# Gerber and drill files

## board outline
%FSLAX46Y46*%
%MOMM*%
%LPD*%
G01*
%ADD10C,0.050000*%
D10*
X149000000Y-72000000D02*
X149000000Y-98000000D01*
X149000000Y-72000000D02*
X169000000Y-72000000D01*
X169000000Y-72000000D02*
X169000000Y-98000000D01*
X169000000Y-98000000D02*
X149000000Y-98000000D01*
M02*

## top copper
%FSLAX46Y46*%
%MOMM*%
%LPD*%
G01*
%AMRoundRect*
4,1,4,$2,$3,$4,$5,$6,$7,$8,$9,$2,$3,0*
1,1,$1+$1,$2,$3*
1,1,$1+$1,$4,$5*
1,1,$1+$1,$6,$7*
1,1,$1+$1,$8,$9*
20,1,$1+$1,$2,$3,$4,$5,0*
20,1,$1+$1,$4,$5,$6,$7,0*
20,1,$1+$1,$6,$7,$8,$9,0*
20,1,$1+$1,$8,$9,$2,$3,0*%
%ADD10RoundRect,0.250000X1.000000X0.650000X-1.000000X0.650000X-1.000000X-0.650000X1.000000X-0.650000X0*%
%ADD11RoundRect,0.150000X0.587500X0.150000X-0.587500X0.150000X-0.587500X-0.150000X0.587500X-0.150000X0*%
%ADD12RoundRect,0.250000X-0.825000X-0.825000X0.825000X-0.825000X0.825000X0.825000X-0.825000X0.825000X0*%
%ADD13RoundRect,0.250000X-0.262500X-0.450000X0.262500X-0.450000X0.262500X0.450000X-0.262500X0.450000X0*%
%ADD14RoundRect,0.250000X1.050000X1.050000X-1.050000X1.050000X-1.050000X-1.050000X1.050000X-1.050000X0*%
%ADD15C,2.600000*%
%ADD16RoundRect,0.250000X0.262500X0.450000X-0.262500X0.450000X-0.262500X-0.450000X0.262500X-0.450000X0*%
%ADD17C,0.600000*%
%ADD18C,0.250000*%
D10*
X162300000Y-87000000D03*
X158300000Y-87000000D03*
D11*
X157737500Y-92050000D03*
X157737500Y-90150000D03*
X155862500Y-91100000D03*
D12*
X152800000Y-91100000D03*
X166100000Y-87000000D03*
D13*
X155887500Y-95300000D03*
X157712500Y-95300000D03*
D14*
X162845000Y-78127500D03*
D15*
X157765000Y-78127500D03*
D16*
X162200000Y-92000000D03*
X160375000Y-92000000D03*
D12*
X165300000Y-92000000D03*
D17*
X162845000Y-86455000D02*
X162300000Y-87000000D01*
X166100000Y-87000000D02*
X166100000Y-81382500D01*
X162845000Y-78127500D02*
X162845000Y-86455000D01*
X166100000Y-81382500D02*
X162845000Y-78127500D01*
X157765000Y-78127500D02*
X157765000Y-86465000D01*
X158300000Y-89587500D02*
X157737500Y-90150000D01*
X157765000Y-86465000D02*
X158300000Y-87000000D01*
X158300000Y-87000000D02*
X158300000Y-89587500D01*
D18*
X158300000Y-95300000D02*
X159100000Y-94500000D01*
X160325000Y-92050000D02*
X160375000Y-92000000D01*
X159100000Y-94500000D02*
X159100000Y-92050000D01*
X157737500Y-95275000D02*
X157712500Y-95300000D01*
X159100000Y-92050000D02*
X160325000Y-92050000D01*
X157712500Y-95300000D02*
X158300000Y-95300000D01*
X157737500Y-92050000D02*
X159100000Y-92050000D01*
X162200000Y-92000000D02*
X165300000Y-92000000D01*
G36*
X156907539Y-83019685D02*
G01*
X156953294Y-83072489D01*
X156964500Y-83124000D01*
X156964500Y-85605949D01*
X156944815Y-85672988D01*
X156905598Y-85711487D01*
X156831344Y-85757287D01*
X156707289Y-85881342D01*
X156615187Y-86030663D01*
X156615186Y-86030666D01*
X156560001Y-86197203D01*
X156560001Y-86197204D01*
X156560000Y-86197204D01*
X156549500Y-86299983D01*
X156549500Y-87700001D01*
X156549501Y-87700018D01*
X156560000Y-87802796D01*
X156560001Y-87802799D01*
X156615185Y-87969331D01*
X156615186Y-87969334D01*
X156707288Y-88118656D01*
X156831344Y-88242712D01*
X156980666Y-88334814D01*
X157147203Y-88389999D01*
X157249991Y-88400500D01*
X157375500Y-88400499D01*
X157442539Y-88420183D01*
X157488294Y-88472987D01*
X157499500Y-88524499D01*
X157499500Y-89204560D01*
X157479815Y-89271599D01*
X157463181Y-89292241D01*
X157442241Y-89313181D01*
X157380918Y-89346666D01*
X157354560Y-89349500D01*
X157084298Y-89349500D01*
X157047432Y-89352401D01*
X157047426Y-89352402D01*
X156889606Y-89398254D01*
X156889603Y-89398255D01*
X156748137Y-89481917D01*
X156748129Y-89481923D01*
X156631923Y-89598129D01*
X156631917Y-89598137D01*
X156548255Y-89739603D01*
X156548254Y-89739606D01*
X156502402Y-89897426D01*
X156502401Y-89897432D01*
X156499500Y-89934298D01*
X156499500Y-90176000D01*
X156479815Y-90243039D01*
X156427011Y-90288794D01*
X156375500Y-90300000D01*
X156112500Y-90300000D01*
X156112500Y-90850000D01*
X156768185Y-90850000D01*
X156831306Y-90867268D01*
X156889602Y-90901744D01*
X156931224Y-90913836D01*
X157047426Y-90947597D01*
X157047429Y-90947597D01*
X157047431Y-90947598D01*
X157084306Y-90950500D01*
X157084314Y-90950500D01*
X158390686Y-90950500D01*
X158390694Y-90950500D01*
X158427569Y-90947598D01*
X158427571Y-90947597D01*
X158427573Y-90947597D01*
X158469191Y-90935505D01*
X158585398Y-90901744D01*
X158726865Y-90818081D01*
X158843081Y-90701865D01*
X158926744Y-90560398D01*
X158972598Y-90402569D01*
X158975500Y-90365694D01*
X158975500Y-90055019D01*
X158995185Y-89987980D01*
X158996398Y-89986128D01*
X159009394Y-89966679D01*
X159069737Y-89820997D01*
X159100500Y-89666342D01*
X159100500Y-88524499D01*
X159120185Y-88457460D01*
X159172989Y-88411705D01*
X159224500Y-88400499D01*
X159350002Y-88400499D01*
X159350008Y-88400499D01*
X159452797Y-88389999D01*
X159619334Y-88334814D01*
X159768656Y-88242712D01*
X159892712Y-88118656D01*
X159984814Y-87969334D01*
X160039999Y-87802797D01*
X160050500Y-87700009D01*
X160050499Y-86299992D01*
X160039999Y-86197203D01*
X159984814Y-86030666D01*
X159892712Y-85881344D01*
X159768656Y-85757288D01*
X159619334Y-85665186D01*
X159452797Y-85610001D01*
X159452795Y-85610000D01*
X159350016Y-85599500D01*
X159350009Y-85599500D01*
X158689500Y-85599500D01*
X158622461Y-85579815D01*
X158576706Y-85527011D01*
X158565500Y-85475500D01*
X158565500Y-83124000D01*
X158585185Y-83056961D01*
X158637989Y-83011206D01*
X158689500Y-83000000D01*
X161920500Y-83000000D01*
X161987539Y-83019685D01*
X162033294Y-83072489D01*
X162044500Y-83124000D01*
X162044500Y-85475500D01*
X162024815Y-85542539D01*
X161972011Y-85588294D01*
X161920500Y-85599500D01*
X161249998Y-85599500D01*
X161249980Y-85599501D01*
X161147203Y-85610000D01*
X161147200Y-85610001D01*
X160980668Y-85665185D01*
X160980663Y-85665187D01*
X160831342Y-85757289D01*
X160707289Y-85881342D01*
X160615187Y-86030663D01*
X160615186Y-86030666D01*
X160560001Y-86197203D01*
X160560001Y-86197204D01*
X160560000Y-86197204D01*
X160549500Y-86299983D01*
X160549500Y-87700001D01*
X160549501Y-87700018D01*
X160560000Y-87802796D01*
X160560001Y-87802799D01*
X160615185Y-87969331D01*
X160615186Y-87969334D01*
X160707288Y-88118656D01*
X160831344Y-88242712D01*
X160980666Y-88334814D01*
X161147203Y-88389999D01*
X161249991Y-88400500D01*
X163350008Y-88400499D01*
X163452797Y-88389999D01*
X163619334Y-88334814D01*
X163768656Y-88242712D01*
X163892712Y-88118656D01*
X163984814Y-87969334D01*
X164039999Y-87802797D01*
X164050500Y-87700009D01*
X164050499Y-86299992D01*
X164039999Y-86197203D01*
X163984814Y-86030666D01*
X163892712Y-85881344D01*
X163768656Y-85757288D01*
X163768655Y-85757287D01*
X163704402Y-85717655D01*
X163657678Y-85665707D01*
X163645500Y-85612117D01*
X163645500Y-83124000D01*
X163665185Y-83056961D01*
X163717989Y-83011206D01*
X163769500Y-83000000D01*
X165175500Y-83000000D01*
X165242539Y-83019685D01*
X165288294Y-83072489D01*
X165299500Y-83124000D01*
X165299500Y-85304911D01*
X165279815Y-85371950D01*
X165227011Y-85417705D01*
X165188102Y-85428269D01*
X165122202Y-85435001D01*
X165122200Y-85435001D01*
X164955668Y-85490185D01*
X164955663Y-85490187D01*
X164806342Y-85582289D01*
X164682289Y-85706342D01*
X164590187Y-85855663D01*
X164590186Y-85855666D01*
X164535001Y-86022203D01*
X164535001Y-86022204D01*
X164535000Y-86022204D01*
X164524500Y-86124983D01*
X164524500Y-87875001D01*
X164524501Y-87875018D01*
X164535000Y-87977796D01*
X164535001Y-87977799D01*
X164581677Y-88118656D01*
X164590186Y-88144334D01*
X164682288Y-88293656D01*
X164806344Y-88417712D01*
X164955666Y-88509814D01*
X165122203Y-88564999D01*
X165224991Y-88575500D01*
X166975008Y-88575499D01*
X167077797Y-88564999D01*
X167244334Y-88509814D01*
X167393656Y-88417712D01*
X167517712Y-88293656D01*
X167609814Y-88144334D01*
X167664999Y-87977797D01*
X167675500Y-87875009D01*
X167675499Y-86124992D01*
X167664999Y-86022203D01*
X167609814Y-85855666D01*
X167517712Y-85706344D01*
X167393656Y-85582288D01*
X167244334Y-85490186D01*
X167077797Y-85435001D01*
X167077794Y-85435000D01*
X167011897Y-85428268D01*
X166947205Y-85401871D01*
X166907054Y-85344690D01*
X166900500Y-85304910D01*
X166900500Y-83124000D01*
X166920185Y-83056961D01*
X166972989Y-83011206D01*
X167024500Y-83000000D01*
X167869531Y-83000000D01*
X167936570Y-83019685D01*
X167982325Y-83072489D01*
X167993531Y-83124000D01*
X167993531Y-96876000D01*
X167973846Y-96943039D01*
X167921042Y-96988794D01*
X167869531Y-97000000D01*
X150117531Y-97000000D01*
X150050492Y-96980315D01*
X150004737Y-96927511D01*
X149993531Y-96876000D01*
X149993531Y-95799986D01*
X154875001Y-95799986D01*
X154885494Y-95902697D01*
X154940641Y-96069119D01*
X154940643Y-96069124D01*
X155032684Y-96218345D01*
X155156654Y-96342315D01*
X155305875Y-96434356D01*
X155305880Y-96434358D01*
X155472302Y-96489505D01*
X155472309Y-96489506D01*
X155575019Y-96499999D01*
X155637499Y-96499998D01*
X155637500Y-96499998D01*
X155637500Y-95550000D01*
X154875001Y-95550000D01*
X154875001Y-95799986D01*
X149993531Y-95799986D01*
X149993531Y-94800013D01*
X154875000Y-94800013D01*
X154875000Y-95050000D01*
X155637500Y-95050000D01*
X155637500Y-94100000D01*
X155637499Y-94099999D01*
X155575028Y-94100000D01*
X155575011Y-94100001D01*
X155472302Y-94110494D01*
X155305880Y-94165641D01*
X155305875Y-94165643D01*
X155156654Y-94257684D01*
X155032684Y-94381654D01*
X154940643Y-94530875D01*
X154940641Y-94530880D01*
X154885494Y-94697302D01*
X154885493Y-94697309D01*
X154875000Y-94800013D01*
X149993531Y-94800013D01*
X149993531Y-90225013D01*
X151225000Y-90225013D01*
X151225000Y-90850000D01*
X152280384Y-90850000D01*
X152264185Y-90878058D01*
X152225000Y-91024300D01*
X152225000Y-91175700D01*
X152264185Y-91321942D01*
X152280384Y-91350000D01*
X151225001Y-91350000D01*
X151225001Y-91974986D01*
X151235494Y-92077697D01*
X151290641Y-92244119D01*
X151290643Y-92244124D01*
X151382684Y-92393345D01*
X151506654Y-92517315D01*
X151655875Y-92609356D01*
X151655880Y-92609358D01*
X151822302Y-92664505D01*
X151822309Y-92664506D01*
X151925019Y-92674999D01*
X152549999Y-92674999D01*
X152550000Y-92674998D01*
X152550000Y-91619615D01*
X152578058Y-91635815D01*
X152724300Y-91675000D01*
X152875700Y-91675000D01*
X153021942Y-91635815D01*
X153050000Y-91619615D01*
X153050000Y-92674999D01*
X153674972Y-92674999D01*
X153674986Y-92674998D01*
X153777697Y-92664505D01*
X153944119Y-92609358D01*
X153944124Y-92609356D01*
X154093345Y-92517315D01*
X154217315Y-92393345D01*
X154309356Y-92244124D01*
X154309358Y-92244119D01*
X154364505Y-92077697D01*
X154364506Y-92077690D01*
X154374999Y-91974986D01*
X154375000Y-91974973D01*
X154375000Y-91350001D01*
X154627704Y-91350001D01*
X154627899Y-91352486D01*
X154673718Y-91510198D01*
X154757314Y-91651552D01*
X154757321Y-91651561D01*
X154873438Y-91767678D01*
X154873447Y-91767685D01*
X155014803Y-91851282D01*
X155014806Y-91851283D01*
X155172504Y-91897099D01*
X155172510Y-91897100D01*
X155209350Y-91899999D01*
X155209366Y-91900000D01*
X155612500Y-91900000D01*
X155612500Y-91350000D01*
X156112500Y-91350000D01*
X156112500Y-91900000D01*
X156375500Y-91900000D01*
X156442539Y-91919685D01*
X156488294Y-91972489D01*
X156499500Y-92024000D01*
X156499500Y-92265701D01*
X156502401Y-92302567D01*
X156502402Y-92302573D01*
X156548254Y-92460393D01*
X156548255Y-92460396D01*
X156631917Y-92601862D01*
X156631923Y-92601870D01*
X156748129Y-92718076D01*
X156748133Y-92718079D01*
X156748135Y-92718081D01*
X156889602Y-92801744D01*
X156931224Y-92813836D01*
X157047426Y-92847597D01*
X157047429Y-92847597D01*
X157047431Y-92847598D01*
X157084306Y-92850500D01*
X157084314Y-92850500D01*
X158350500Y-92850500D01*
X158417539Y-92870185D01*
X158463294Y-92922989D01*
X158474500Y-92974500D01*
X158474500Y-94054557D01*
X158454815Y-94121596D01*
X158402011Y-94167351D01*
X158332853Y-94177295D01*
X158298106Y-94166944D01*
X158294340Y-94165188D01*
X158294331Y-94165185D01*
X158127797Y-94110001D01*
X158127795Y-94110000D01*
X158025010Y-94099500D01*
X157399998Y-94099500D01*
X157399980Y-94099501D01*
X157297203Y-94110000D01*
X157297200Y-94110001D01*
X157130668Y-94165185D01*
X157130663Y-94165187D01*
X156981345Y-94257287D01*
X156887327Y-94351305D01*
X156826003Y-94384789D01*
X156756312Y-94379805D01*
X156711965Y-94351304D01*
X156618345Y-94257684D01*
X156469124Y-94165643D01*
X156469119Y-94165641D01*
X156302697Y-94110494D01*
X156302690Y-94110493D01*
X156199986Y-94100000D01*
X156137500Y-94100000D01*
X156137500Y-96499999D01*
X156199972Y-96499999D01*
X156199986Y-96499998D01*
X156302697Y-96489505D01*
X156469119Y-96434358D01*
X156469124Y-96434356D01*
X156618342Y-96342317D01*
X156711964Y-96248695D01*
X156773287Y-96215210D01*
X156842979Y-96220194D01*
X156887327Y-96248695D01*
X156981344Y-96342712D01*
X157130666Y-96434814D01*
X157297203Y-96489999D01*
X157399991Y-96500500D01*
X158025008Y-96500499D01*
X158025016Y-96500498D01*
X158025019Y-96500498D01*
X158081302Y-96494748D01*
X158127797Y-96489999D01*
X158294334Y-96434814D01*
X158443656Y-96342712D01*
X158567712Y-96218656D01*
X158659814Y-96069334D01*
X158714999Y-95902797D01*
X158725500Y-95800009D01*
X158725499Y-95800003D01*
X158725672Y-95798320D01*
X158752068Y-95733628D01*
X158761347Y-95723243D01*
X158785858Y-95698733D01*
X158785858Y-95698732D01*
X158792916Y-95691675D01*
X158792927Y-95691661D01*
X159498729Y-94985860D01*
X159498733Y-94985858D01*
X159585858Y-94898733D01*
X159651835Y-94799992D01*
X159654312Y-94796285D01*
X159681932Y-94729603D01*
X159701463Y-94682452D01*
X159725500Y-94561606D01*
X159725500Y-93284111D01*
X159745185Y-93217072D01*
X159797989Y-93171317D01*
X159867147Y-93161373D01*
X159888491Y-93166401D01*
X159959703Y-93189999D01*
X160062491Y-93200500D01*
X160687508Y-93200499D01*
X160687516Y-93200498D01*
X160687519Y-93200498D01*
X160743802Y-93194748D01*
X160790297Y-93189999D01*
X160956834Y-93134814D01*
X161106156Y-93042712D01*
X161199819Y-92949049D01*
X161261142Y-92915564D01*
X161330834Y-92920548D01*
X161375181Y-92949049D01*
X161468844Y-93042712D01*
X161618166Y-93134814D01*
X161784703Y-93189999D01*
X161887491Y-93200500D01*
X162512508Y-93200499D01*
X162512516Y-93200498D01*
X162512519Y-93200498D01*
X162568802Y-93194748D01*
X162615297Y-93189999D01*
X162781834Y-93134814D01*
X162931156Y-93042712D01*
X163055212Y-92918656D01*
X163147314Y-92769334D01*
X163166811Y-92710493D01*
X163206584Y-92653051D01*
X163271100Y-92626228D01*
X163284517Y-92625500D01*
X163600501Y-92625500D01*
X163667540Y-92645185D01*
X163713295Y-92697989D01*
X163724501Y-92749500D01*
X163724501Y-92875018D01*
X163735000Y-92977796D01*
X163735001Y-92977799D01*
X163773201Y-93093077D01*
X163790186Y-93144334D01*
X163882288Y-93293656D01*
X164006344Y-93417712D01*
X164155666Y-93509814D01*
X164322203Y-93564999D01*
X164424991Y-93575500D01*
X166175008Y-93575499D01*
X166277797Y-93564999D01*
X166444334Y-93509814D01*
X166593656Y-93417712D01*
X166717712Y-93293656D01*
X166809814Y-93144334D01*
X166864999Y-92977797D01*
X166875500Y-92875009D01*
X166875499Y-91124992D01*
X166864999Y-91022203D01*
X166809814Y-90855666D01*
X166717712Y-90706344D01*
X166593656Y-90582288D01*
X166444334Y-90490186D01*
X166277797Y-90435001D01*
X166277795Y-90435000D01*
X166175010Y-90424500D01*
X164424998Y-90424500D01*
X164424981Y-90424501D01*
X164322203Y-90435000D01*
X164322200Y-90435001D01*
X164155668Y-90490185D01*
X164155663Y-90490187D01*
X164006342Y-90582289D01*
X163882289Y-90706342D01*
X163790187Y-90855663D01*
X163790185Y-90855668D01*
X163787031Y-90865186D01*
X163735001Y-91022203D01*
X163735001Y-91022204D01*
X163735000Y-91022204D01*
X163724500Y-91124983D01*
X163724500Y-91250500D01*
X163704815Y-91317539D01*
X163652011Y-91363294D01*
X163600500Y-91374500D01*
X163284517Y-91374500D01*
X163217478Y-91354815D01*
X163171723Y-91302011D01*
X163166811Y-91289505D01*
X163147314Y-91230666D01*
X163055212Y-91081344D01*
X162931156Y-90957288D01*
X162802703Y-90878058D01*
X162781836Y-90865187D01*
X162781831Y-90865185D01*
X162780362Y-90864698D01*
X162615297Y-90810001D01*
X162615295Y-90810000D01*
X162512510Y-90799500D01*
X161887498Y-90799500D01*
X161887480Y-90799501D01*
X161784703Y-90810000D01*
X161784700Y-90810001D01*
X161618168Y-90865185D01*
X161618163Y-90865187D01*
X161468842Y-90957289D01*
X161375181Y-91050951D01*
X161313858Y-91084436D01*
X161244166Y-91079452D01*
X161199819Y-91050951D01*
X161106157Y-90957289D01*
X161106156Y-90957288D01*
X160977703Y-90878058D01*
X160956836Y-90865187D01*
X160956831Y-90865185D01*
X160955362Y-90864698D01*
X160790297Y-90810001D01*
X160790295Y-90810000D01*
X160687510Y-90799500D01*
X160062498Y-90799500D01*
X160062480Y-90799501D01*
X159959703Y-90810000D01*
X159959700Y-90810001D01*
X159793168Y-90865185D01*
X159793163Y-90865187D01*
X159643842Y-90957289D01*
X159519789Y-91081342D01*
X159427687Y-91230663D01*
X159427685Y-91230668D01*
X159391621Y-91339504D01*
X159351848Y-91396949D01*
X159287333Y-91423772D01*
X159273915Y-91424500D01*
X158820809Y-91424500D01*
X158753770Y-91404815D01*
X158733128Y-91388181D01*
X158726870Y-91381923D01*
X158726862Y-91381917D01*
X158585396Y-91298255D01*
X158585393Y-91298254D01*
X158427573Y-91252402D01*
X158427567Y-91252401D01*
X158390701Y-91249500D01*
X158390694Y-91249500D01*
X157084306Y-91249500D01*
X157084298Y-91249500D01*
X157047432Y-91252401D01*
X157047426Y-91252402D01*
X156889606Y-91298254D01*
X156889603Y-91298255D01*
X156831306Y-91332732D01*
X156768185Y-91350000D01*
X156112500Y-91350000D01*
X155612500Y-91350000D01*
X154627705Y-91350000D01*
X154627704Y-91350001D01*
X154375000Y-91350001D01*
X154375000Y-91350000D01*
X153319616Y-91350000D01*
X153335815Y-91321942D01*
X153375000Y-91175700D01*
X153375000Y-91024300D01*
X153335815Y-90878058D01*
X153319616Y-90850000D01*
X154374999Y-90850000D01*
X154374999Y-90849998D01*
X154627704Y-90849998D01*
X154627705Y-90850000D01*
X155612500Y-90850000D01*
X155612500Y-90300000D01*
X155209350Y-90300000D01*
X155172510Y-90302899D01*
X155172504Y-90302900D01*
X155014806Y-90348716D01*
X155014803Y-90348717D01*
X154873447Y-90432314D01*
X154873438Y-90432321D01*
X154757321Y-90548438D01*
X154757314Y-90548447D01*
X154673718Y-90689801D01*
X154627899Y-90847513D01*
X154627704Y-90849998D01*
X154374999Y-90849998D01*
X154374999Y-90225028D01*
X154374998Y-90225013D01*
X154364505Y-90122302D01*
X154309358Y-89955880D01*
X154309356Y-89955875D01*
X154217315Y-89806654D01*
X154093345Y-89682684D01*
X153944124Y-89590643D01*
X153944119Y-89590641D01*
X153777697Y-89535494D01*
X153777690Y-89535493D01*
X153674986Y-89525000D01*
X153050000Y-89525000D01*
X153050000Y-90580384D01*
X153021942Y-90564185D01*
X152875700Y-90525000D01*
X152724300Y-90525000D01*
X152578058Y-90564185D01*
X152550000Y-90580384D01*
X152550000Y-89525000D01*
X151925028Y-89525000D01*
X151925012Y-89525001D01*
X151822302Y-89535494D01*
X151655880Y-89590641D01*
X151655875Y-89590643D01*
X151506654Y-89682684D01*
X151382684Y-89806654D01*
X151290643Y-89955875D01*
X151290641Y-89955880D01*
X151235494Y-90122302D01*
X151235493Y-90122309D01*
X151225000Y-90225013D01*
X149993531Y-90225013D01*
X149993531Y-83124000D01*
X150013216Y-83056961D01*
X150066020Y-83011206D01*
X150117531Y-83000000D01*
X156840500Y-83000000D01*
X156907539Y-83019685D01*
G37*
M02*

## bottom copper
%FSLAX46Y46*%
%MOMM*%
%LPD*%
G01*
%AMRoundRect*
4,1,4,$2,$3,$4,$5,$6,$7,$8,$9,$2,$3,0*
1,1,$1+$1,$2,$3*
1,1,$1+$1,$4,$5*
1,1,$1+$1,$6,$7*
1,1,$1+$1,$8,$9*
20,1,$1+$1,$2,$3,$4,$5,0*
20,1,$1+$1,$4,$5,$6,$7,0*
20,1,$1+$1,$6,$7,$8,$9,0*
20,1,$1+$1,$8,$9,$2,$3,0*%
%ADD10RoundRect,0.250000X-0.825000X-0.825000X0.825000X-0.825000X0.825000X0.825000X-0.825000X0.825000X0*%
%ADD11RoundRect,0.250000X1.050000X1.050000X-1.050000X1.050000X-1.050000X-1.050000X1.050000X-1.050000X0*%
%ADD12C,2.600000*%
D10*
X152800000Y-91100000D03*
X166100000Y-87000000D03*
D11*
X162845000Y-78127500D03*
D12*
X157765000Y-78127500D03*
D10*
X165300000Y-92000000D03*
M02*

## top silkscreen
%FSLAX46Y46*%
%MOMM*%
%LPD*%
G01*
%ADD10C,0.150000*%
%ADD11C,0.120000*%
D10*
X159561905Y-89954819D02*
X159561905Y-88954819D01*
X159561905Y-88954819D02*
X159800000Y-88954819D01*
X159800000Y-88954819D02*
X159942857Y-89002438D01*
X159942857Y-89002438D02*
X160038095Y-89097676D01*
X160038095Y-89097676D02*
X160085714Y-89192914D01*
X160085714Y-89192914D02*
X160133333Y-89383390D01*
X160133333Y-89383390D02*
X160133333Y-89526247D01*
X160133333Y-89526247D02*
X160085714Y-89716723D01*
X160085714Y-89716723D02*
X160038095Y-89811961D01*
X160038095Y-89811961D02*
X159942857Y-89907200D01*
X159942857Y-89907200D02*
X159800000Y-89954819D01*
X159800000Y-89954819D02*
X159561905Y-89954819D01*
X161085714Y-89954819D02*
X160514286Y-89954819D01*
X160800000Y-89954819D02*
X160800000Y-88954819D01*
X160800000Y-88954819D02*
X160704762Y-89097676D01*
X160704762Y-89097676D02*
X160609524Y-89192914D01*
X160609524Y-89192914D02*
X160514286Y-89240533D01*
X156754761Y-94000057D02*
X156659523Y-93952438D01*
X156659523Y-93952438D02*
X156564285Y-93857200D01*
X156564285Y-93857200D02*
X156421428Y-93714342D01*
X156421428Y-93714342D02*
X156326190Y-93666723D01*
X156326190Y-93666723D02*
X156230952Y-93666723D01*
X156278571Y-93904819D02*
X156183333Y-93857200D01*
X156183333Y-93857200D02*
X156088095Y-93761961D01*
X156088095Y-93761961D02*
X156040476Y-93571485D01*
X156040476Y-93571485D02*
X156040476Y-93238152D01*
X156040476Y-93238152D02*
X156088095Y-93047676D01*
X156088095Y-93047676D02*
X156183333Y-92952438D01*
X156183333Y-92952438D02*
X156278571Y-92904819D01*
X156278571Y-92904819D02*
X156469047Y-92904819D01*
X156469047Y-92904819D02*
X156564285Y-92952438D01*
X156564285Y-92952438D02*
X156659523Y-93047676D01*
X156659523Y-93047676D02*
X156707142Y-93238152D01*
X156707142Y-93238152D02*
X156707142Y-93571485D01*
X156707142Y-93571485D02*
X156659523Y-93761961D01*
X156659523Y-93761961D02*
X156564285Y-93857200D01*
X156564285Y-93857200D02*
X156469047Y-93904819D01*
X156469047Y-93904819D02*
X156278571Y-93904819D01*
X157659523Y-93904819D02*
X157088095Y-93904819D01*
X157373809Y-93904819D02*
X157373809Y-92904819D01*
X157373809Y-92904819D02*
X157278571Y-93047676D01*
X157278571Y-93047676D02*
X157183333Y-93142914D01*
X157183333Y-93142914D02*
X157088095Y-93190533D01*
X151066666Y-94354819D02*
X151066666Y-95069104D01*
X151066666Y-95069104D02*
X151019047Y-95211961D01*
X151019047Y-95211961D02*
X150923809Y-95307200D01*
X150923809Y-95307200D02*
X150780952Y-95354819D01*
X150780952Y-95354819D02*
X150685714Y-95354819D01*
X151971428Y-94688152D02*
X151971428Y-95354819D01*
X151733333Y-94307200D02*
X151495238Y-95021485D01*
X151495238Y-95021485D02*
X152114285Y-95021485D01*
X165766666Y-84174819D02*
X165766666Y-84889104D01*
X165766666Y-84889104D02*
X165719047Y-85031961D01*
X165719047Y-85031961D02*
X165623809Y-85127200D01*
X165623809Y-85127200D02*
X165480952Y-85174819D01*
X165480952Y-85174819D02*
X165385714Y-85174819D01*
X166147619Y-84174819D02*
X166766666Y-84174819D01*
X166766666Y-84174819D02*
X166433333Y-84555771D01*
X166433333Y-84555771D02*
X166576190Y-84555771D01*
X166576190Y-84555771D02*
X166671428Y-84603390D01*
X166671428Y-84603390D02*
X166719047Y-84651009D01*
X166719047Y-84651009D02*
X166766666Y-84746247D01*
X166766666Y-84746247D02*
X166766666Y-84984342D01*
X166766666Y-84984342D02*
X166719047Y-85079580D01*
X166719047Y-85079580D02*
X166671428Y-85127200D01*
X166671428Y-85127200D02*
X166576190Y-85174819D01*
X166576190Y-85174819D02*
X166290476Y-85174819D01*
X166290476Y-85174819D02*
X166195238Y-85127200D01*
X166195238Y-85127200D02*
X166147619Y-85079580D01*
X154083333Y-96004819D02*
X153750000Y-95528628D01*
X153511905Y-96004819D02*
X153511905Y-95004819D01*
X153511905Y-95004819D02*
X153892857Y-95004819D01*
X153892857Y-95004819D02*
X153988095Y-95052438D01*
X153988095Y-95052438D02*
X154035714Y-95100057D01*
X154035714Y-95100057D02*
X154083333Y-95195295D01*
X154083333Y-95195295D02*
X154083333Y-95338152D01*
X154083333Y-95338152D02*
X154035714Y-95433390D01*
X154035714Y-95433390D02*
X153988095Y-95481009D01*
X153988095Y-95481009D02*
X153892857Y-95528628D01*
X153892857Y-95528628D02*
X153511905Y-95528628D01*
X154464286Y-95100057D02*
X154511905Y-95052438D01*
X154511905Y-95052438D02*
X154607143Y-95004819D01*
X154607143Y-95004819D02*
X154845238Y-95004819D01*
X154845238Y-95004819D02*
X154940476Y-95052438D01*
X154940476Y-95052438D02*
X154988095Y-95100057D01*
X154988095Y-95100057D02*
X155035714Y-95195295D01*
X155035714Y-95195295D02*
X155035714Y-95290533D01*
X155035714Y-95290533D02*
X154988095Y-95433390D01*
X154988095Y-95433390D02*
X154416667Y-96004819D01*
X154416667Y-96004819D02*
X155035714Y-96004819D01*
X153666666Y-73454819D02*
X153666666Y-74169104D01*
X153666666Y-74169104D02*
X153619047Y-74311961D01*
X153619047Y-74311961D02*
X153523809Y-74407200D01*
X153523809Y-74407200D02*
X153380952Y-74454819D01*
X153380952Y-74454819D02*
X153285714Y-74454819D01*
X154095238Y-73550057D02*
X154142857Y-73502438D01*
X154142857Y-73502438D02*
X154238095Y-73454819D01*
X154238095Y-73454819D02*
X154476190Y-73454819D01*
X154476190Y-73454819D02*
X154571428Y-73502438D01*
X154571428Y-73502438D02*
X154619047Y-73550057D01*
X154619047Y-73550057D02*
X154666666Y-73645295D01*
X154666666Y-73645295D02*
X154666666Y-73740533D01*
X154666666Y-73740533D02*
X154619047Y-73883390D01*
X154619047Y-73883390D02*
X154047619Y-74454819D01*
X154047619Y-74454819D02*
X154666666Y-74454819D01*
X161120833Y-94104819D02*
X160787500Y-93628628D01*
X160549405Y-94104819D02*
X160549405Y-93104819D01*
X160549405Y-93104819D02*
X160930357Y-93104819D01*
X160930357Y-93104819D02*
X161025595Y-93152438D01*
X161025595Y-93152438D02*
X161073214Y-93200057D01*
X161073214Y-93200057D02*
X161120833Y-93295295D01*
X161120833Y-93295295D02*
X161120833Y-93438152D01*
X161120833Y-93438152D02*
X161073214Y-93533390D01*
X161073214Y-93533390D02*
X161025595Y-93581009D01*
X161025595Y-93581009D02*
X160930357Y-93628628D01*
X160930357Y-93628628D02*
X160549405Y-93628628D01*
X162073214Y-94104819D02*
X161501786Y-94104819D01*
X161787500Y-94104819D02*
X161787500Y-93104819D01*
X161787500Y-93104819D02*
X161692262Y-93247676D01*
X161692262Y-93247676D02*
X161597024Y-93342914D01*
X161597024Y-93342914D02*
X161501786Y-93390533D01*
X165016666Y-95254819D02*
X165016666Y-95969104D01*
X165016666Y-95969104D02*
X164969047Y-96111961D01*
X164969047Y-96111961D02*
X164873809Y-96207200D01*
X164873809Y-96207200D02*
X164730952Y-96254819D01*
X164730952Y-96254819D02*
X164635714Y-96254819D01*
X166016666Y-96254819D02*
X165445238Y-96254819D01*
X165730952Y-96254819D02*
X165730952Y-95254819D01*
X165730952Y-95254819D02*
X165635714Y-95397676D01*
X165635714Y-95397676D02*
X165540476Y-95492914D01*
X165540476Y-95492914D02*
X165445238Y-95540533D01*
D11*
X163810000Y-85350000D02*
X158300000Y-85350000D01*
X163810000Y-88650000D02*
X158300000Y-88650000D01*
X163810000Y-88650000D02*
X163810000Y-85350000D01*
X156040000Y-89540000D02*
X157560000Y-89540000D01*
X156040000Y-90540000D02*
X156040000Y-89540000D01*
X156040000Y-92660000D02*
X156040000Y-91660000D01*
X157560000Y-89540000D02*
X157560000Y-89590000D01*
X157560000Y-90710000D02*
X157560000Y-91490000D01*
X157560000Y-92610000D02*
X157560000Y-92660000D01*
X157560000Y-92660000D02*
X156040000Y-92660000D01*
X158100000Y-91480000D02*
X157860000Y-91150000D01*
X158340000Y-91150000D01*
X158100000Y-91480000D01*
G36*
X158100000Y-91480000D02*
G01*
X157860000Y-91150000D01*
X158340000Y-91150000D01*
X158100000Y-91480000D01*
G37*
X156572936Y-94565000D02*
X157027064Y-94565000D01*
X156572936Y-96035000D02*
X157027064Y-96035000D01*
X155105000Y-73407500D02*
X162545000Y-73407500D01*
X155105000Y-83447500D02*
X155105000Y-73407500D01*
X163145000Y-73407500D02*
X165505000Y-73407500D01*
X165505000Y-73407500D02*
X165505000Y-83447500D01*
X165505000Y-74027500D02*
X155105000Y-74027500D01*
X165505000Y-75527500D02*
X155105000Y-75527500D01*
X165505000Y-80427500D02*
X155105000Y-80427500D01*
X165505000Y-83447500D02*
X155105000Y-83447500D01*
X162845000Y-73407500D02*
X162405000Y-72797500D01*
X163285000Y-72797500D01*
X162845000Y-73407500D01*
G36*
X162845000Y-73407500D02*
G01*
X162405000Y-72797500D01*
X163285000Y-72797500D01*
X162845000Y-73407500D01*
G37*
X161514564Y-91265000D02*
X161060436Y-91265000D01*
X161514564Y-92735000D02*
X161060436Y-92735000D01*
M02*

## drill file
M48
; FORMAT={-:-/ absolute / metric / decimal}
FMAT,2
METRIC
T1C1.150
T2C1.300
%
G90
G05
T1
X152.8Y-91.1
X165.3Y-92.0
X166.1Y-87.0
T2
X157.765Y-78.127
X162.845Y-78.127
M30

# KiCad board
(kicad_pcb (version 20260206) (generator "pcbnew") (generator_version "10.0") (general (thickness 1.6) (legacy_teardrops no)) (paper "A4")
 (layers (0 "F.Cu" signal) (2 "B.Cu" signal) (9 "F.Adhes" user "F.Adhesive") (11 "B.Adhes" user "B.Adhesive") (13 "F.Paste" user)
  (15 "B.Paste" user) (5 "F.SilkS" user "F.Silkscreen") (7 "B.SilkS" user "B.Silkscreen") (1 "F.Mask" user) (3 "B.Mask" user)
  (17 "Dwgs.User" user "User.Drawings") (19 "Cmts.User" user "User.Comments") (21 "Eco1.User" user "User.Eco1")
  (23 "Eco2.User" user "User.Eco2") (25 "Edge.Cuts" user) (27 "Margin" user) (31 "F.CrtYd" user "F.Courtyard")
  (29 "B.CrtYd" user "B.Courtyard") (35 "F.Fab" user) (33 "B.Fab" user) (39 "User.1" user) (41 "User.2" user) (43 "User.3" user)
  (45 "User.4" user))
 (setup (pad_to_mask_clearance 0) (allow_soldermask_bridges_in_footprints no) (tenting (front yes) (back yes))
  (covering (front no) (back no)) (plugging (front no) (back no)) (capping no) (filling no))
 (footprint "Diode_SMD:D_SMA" (layer "F.Cu") (at 160.3 87 180)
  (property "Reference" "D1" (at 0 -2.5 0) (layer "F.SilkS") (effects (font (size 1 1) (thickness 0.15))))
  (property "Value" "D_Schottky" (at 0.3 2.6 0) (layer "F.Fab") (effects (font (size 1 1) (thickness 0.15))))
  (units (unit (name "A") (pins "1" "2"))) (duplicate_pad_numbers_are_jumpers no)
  (fp_line (start -3.51 1.65) (end 2 1.65) (stroke (width 0.12) (type solid)) (layer "F.SilkS"))
  (fp_line (start -3.51 -1.65) (end 2 -1.65) (stroke (width 0.12) (type solid)) (layer "F.SilkS"))
  (fp_line (start -3.51 -1.65) (end -3.51 1.65) (stroke (width 0.12) (type solid)) (layer "F.SilkS"))
  (pad "1" smd roundrect (at -2 0 180) (size 2.5 1.8) (layers "F.Cu" "F.Mask" "F.Paste") (roundrect_rratio 0.1388888889) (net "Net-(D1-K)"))
  (pad "2" smd roundrect (at 2 0 180) (size 2.5 1.8) (layers "F.Cu" "F.Mask" "F.Paste") (roundrect_rratio 0.1388888889) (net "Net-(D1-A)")))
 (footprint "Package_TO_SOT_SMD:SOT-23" (layer "F.Cu") (at 156.8 91.1 180)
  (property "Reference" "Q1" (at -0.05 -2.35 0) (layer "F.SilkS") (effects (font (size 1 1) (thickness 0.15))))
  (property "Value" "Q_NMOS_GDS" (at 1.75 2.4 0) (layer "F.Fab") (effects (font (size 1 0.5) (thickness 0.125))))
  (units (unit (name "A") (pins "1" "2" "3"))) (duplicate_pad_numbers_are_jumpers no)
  (fp_line (start 0.76 1.56) (end -0.76 1.56) (stroke (width 0.12) (type solid)) (layer "F.SilkS"))
  (fp_line (start 0.76 0.56) (end 0.76 1.56) (stroke (width 0.12) (type solid)) (layer "F.SilkS"))
  (fp_line (start 0.76 -1.56) (end 0.76 -0.56) (stroke (width 0.12) (type solid)) (layer "F.SilkS"))
  (fp_line (start -0.76 1.56) (end -0.76 1.51) (stroke (width 0.12) (type solid)) (layer "F.SilkS"))
  (fp_line (start -0.76 0.39) (end -0.76 -0.39) (stroke (width 0.12) (type solid)) (layer "F.SilkS"))
  (fp_line (start -0.76 -1.51) (end -0.76 -1.56) (stroke (width 0.12) (type solid)) (layer "F.SilkS"))
  (fp_line (start -0.76 -1.56) (end 0.76 -1.56) (stroke (width 0.12) (type solid)) (layer "F.SilkS"))
  (fp_poly (pts (xy -1.3 -0.38) (xy -1.06 -0.05) (xy -1.54 -0.05)) (stroke (width 0.12) (type solid)) (fill yes) (layer "F.SilkS"))
  (pad "1" smd roundrect (at -0.9375 -0.95 180) (size 1.475 0.6) (layers "F.Cu" "F.Mask" "F.Paste") (roundrect_rratio 0.25)
   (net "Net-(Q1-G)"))
  (pad "2" smd roundrect (at -0.9375 0.95 180) (size 1.475 0.6) (layers "F.Cu" "F.Mask" "F.Paste") (roundrect_rratio 0.25)
   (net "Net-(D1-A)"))
  (pad "3" smd roundrect (at 0.9375 0 180) (size 1.475 0.6) (layers "F.Cu" "F.Mask" "F.Paste") (roundrect_rratio 0.25) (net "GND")))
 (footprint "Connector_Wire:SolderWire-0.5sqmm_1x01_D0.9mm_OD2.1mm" (layer "F.Cu") (at 152.8 91.1)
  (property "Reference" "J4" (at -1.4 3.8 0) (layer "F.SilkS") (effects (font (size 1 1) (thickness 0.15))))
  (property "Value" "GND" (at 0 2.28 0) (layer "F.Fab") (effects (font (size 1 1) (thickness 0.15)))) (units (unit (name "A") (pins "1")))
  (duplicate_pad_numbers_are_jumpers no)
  (pad "1" thru_hole roundrect (at 0 0) (size 2.15 2.15) (drill 1.15) (layers "*.Cu" "*.Mask") (remove_unused_layers no)
   (roundrect_rratio 0.116279) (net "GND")))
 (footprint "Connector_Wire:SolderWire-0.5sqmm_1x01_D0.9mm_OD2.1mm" (layer "F.Cu") (at 166.1 87)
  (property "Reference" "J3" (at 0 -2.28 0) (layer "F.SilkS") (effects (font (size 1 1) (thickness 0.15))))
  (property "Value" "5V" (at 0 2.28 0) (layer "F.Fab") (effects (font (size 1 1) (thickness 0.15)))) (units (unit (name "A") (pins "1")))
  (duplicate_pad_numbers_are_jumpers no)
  (pad "1" thru_hole roundrect (at 0 0) (size 2.15 2.15) (drill 1.15) (layers "*.Cu" "*.Mask") (remove_unused_layers no)
   (roundrect_rratio 0.116279) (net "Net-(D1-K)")))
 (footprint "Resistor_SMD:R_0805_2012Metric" (layer "F.Cu") (at 156.8 95.3)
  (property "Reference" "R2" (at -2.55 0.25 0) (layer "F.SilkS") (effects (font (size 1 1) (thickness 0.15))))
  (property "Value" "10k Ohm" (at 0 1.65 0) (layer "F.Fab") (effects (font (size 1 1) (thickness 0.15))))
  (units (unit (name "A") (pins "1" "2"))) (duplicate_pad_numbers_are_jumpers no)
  (fp_line (start -0.227064 -0.735) (end 0.227064 -0.735) (stroke (width 0.12) (type solid)) (layer "F.SilkS"))
  (fp_line (start -0.227064 0.735) (end 0.227064 0.735) (stroke (width 0.12) (type solid)) (layer "F.SilkS"))
  (pad "1" smd roundrect (at -0.9125 0) (size 1.025 1.4) (layers "F.Cu" "F.Mask" "F.Paste") (roundrect_rratio 0.243902) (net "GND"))
  (pad "2" smd roundrect (at 0.9125 0) (size 1.025 1.4) (layers "F.Cu" "F.Mask" "F.Paste") (roundrect_rratio 0.243902) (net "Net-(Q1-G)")))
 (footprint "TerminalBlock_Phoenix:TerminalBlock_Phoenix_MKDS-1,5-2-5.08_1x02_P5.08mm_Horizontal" (layer "F.Cu") (at 162.845 78.1275 180)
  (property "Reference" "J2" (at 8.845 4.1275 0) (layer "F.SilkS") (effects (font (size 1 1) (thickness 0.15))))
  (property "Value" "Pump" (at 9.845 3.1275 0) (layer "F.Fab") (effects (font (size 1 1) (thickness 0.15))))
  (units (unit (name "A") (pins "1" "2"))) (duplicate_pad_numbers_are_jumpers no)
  (fp_line (start 7.74 4.72) (end 0.3 4.72) (stroke (width 0.12) (type solid)) (layer "F.SilkS"))
  (fp_line (start 7.74 -5.32) (end 7.74 4.72) (stroke (width 0.12) (type solid)) (layer "F.SilkS"))
  (fp_line (start -0.3 4.72) (end -2.66 4.72) (stroke (width 0.12) (type solid)) (layer "F.SilkS"))
  (fp_line (start -2.66 4.72) (end -2.66 -5.32) (stroke (width 0.12) (type solid)) (layer "F.SilkS"))
  (fp_line (start -2.66 4.1) (end 7.74 4.1) (stroke (width 0.12) (type solid)) (layer "F.SilkS"))
  (fp_line (start -2.66 2.6) (end 7.74 2.6) (stroke (width 0.12) (type solid)) (layer "F.SilkS"))
  (fp_line (start -2.66 -2.3) (end 7.74 -2.3) (stroke (width 0.12) (type solid)) (layer "F.SilkS"))
  (fp_line (start -2.66 -5.32) (end 7.74 -5.32) (stroke (width 0.12) (type solid)) (layer "F.SilkS"))
  (fp_poly (pts (xy 0 4.72) (xy 0.44 5.33) (xy -0.44 5.33)) (stroke (width 0.12) (type solid)) (fill yes) (layer "F.SilkS"))
  (pad "1" thru_hole roundrect (at 0 0 180) (size 2.6 2.6) (drill 1.3) (layers "*.Cu" "*.Mask") (remove_unused_layers no)
   (roundrect_rratio 0.096154) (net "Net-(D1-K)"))
  (pad "2" thru_hole circle (at 5.08 0 180) (size 2.6 2.6) (drill 1.3) (layers "*.Cu" "*.Mask") (remove_unused_layers no) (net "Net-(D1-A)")))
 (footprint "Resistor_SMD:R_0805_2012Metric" (layer "F.Cu") (at 161.2875 92 180)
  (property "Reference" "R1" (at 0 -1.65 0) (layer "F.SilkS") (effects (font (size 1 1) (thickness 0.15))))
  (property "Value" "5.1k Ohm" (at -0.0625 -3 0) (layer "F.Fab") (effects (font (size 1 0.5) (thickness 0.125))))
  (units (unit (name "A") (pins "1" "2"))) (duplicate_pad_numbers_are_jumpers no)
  (fp_line (start -0.227064 0.735) (end 0.227064 0.735) (stroke (width 0.12) (type solid)) (layer "F.SilkS"))
  (fp_line (start -0.227064 -0.735) (end 0.227064 -0.735) (stroke (width 0.12) (type solid)) (layer "F.SilkS"))
  (pad "1" smd roundrect (at -0.9125 0 180) (size 1.025 1.4) (layers "F.Cu" "F.Mask" "F.Paste") (roundrect_rratio 0.243902)
   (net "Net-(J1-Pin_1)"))
  (pad "2" smd roundrect (at 0.9125 0 180) (size 1.025 1.4) (layers "F.Cu" "F.Mask" "F.Paste") (roundrect_rratio 0.243902)
   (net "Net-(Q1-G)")))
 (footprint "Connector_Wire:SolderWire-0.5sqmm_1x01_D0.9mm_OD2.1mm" (layer "F.Cu") (at 165.3 92)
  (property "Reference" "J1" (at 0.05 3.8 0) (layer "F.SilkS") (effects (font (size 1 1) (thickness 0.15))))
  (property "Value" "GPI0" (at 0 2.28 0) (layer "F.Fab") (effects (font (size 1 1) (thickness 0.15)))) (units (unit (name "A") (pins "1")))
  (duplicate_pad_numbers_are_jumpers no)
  (pad "1" thru_hole roundrect (at 0 0) (size 2.15 2.15) (drill 1.15) (layers "*.Cu" "*.Mask") (remove_unused_layers no)
   (roundrect_rratio 0.116279) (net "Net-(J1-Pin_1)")))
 (gr_line (start 149 72) (end 149 98) (stroke (width 0.05) (type default)) (layer "Edge.Cuts"))
 (gr_line (start 149 72) (end 169 72) (stroke (width 0.05) (type default)) (layer "Edge.Cuts"))
 (gr_line (start 169 72) (end 169 98) (stroke (width 0.05) (type default)) (layer "Edge.Cuts"))
 (gr_line (start 169 98) (end 149 98) (stroke (width 0.05) (type default)) (layer "Edge.Cuts"))
 (segment (start 162.845 86.455) (end 162.3 87) (width 0.6) (layer "F.Cu") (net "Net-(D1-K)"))
 (segment (start 166.1 87) (end 166.1 81.3825) (width 0.6) (layer "F.Cu") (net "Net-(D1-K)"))
 (segment (start 162.845 78.1275) (end 162.845 86.455) (width 0.6) (layer "F.Cu") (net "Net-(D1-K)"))
 (segment (start 166.1 81.3825) (end 162.845 78.1275) (width 0.6) (layer "F.Cu") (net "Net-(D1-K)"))
 (segment (start 157.765 78.1275) (end 157.765 86.465) (width 0.6) (layer "F.Cu") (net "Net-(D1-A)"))
 (segment (start 158.3 89.5875) (end 157.7375 90.15) (width 0.6) (layer "F.Cu") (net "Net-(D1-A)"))
 (segment (start 157.765 86.465) (end 158.3 87) (width 0.6) (layer "F.Cu") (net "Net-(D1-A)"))
 (segment (start 158.3 87) (end 158.3 89.5875) (width 0.6) (layer "F.Cu") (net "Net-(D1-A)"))
 (segment (start 158.3 95.3) (end 159.1 94.5) (width 0.25) (layer "F.Cu") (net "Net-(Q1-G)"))
 (segment (start 160.325 92.05) (end 160.375 92) (width 0.25) (layer "F.Cu") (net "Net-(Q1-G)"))
 (segment (start 159.1 94.5) (end 159.1 92.05) (width 0.25) (layer "F.Cu") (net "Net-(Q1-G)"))
 (segment (start 157.7375 95.275) (end 157.7125 95.3) (width 0.25) (layer "F.Cu") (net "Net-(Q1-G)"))
 (segment (start 159.1 92.05) (end 160.325 92.05) (width 0.25) (layer "F.Cu") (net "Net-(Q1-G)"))
 (segment (start 157.7125 95.3) (end 158.3 95.3) (width 0.25) (layer "F.Cu") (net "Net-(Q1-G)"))
 (segment (start 157.7375 92.05) (end 159.1 92.05) (width 0.25) (layer "F.Cu") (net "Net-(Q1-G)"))
 (segment (start 162.2 92) (end 165.3 92) (width 0.25) (layer "F.Cu") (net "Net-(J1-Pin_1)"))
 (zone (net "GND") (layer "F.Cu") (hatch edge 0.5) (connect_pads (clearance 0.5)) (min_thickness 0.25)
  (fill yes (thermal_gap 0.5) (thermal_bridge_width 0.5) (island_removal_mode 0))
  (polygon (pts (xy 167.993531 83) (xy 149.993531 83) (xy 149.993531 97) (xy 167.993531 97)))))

